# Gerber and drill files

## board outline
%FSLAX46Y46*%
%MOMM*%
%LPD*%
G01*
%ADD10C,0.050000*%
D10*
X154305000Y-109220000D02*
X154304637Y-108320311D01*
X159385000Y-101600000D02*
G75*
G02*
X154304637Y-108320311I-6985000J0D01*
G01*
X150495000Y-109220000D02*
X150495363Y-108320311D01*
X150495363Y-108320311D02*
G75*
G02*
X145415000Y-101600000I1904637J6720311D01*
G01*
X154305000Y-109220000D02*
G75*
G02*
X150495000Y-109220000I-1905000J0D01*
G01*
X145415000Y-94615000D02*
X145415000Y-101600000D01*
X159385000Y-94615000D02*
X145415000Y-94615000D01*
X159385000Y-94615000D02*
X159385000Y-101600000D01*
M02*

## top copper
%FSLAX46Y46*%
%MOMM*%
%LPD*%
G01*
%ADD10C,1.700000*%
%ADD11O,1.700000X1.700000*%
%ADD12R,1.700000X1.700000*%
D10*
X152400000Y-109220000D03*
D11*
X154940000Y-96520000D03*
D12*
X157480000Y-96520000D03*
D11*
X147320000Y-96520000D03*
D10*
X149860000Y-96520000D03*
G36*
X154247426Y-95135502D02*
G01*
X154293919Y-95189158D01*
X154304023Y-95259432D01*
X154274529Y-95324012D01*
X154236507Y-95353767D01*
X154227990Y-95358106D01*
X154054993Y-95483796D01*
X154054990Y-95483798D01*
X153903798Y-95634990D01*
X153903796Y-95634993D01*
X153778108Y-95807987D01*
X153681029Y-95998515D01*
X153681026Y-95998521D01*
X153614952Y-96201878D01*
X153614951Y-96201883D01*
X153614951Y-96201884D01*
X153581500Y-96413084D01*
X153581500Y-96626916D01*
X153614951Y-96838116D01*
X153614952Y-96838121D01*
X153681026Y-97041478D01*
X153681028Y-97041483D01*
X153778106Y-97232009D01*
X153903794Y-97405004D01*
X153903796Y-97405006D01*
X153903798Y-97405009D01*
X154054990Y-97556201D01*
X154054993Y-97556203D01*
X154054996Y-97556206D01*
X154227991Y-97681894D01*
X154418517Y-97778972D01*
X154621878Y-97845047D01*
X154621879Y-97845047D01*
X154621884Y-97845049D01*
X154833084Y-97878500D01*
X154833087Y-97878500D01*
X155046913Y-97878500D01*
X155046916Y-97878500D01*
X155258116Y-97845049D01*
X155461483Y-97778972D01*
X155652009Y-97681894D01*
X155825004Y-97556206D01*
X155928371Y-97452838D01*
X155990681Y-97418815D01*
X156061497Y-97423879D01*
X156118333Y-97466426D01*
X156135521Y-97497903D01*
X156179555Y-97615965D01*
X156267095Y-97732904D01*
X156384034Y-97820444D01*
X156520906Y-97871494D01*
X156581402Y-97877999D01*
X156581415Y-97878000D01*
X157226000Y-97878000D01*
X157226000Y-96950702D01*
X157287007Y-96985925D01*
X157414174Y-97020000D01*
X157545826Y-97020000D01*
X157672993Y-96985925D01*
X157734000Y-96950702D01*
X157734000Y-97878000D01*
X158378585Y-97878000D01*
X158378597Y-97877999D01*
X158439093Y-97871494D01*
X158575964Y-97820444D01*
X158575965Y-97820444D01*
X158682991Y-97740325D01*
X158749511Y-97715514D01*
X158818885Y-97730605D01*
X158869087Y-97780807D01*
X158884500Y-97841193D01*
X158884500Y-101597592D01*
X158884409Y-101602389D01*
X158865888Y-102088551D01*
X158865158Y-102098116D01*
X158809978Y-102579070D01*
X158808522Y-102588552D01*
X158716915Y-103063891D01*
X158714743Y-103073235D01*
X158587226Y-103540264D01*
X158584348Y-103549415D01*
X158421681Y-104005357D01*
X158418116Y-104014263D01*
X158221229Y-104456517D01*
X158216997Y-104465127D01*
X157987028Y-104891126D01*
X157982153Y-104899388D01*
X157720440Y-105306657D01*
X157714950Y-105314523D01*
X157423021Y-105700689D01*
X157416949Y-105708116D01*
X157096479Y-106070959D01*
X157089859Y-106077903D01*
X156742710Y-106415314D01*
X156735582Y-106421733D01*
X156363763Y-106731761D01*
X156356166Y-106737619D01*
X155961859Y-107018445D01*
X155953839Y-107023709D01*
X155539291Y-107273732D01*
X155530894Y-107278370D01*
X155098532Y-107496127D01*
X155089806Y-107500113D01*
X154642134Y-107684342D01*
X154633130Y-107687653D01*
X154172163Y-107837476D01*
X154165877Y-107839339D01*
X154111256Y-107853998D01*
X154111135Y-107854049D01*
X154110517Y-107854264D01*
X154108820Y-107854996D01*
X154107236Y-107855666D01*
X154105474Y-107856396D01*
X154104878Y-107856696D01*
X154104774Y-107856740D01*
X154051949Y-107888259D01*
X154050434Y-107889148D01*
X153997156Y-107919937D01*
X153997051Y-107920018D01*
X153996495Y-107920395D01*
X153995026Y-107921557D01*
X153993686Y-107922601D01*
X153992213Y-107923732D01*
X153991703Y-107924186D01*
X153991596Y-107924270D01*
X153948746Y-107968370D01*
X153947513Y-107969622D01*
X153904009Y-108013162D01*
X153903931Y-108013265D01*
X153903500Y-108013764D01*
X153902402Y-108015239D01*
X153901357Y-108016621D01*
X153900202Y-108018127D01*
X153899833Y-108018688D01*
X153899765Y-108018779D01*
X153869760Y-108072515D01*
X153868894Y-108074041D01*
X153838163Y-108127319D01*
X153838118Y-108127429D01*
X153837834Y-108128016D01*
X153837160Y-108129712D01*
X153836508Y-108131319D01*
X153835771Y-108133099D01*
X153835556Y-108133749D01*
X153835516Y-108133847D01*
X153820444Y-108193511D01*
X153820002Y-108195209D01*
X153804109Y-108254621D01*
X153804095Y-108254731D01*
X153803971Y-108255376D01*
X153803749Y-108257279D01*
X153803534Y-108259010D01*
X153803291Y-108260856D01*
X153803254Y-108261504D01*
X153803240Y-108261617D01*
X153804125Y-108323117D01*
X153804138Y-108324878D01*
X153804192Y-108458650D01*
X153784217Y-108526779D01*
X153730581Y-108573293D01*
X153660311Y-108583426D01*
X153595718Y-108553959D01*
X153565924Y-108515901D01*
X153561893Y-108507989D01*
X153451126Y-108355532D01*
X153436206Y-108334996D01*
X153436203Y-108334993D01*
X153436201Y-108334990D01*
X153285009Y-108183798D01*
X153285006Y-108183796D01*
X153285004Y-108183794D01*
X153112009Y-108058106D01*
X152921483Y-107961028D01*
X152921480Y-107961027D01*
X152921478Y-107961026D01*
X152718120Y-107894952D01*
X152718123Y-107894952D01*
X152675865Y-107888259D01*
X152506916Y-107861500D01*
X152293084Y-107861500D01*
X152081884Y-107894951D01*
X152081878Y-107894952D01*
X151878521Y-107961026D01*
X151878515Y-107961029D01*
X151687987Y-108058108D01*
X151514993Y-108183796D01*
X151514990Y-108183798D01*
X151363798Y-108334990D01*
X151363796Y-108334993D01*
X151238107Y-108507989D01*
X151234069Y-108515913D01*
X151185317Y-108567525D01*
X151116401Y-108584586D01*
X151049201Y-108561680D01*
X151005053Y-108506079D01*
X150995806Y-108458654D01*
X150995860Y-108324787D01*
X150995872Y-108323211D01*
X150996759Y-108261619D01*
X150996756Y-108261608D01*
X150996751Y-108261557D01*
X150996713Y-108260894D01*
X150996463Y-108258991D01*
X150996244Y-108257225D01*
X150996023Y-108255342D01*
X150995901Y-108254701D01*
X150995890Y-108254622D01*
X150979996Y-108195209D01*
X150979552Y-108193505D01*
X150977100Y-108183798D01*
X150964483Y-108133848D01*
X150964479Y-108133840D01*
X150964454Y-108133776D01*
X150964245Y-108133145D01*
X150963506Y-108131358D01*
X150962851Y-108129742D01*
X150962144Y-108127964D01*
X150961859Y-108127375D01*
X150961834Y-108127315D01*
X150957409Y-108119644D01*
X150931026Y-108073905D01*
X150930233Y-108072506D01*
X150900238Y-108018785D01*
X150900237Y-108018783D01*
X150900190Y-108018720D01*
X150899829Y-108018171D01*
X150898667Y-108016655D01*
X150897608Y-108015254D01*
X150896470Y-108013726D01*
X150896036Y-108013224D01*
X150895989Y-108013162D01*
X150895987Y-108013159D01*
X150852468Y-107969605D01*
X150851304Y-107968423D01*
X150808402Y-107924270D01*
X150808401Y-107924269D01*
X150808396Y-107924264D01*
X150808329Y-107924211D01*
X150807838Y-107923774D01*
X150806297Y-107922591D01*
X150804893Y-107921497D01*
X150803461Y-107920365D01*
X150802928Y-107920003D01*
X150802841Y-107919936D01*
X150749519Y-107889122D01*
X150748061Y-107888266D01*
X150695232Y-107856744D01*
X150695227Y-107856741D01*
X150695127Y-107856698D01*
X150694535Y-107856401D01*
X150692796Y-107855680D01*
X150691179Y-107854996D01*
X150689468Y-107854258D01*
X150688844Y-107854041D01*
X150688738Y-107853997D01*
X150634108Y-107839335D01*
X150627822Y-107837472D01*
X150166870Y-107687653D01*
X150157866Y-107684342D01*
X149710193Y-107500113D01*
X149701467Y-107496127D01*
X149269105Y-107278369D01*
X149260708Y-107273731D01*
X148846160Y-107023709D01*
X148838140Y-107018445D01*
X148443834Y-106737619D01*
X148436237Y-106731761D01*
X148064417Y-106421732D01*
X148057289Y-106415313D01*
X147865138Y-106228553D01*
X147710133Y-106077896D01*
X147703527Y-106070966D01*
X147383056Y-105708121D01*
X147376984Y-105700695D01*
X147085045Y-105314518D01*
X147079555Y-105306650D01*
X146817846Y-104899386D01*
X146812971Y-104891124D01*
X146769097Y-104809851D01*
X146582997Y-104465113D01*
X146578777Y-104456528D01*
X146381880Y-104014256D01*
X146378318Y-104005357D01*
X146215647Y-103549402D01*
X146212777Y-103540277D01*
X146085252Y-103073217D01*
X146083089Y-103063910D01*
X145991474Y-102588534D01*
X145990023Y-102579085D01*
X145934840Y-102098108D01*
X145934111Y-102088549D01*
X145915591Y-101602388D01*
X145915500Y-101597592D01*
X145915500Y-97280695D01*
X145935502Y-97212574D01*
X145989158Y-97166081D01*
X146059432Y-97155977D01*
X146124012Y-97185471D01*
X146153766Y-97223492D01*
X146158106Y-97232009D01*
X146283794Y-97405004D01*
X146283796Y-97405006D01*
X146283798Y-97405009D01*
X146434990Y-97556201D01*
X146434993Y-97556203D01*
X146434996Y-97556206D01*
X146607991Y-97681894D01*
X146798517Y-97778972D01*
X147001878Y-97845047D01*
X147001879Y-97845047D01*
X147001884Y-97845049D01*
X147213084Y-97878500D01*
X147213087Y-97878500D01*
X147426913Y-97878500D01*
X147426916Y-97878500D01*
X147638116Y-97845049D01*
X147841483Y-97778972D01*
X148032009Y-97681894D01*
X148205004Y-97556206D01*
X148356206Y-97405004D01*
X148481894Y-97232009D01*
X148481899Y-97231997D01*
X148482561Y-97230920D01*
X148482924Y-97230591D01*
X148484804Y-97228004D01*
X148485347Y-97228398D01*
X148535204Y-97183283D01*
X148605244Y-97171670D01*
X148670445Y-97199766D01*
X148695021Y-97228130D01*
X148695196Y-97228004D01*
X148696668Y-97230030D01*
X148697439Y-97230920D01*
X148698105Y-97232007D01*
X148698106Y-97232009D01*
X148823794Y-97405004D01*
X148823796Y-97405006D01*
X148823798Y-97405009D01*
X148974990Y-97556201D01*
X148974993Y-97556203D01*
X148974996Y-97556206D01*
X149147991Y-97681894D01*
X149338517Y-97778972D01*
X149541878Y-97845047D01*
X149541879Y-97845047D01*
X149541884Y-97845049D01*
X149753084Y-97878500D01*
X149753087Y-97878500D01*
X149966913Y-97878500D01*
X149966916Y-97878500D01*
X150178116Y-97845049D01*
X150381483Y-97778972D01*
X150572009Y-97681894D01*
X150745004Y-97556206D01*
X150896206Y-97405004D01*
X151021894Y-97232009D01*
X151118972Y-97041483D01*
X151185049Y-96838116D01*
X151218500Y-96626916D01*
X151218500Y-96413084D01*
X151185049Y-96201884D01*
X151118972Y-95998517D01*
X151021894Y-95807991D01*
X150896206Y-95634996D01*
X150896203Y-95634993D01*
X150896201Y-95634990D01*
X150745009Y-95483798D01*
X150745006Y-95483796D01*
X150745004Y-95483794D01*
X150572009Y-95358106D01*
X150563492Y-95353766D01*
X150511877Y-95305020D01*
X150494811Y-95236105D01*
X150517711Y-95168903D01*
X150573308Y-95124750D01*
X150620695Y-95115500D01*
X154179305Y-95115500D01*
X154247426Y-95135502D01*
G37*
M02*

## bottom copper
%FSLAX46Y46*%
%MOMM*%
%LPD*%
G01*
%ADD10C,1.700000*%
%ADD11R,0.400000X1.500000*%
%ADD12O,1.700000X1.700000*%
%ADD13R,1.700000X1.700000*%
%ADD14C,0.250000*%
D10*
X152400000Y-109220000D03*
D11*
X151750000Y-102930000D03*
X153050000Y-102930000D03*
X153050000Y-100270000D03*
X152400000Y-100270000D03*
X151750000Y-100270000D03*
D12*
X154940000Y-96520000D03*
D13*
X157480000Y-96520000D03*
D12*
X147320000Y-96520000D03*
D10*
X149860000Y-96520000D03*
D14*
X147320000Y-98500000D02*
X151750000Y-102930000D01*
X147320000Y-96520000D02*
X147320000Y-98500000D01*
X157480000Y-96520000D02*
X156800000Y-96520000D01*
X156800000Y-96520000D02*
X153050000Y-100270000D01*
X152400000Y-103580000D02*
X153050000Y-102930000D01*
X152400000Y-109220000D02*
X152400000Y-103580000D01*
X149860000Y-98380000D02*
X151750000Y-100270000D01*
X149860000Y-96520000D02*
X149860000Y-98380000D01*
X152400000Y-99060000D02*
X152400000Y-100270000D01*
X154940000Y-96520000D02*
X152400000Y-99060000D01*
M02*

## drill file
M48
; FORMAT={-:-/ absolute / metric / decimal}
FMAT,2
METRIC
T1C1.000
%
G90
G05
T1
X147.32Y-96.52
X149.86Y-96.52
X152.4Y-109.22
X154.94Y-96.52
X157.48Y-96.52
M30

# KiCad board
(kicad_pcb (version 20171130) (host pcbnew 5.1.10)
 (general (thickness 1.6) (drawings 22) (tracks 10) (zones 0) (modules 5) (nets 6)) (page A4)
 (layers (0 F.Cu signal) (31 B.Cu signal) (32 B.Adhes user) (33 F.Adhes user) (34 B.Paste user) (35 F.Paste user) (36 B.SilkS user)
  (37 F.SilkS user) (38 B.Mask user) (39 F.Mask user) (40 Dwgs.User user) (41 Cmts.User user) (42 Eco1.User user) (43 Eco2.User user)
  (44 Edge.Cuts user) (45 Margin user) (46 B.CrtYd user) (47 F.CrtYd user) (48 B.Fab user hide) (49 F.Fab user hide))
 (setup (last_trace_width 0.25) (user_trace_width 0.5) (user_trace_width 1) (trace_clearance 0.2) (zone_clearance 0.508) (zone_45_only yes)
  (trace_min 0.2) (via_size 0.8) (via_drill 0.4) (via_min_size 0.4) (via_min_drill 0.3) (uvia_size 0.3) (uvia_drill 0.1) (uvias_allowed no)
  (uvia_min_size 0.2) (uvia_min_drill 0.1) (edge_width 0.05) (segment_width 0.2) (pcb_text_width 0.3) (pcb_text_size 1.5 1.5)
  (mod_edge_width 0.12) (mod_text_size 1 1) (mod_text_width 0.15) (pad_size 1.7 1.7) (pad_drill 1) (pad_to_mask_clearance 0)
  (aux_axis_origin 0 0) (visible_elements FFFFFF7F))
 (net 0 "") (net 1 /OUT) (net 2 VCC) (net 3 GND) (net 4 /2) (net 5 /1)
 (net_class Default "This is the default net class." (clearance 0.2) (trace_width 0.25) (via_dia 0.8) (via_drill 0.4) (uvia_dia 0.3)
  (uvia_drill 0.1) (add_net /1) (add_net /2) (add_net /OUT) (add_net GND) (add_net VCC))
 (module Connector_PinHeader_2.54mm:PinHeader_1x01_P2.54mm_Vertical (layer B.Cu) (at 152.4 109.22 270)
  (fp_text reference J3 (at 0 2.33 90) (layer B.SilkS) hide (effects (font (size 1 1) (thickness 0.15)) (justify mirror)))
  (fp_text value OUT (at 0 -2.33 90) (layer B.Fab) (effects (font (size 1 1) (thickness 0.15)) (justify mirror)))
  (pad 1 thru_hole circle (at 0 0 270) (size 1.7 1.7) (drill 1) (layers *.Cu *.Mask) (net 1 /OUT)))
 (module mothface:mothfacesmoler (layer B.Cu) (at 155.575 102.87 255)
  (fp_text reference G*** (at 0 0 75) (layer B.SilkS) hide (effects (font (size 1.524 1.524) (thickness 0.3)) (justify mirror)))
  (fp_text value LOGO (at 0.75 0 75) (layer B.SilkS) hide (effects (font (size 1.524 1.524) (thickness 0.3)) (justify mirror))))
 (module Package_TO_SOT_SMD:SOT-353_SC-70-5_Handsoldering (layer B.Cu) (at 152.4 101.6 270)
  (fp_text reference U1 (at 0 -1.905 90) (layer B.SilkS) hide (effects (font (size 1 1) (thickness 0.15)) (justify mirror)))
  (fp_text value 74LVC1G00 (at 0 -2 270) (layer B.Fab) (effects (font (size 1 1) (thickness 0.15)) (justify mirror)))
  (pad 5 smd rect (at 1.33 0.65 270) (size 1.5 0.4) (layers B.Cu B.Paste B.Mask) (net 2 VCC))
  (pad 4 smd rect (at 1.33 -0.65 270) (size 1.5 0.4) (layers B.Cu B.Paste B.Mask) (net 1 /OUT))
  (pad 3 smd rect (at -1.33 -0.65 270) (size 1.5 0.4) (layers B.Cu B.Paste B.Mask) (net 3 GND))
  (pad 2 smd rect (at -1.33 0 270) (size 1.5 0.4) (layers B.Cu B.Paste B.Mask) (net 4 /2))
  (pad 1 smd rect (at -1.33 0.65 270) (size 1.5 0.4) (layers B.Cu B.Paste B.Mask) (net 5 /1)))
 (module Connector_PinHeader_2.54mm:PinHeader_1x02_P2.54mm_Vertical (layer B.Cu) (at 157.48 96.52 90)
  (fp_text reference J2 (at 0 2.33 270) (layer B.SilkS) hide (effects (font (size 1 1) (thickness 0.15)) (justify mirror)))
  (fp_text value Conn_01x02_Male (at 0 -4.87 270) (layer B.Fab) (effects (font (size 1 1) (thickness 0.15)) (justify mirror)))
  (pad 2 thru_hole oval (at 0 -2.54 90) (size 1.7 1.7) (drill 1) (layers *.Cu *.Mask) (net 4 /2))
  (pad 1 thru_hole rect (at 0 0 90) (size 1.7 1.7) (drill 1) (layers *.Cu *.Mask) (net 3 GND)))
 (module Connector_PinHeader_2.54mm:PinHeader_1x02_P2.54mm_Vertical (layer B.Cu) (at 149.86 96.52 90)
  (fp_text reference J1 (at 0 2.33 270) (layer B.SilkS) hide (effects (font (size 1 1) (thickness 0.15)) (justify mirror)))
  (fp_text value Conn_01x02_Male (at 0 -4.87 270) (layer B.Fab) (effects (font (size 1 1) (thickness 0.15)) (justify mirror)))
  (pad 2 thru_hole oval (at 0 -2.54 90) (size 1.7 1.7) (drill 1) (layers *.Cu *.Mask) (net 2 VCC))
  (pad 1 thru_hole circle (at 0 0 90) (size 1.7 1.7) (drill 1) (layers *.Cu *.Mask) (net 5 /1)))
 (gr_line (start 154.305 109.22) (end 154.304637 108.320311) (layer Edge.Cuts) (width 0.05))
 (gr_arc (start 152.4 101.6) (end 159.385 101.6) (angle 74.17647245) (layer Edge.Cuts) (width 0.05))
 (gr_line (start 150.495 109.22) (end 150.495363 108.320311) (layer Edge.Cuts) (width 0.05))
 (gr_arc (start 152.4 101.6) (end 145.415 101.6) (angle -74.17647245) (layer Edge.Cuts) (width 0.05))
 (gr_arc (start 152.4 109.22) (end 150.495 109.22) (angle -180) (layer Edge.Cuts) (width 0.05))
 (gr_line (start 145.415 94.615) (end 145.415 101.6) (layer Edge.Cuts) (width 0.05))
 (gr_line (start 159.385 94.615) (end 145.415 94.615) (layer Edge.Cuts) (width 0.05))
 (gr_line (start 159.385 94.615) (end 159.385 101.6) (layer Edge.Cuts) (width 0.05))
 (segment (start 147.32 98.5) (end 151.75 102.93) (width 0.25) (layer B.Cu) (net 2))
 (segment (start 147.32 96.52) (end 147.32 98.5) (width 0.25) (layer B.Cu) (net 2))
 (segment (start 157.48 96.52) (end 156.8 96.52) (width 0.25) (layer B.Cu) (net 3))
 (segment (start 156.8 96.52) (end 153.05 100.27) (width 0.25) (layer B.Cu) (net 3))
 (segment (start 152.4 103.58) (end 153.05 102.93) (width 0.25) (layer B.Cu) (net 1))
 (segment (start 152.4 109.22) (end 152.4 103.58) (width 0.25) (layer B.Cu) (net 1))
 (segment (start 149.86 98.38) (end 151.75 100.27) (width 0.25) (layer B.Cu) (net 5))
 (segment (start 149.86 96.52) (end 149.86 98.38) (width 0.25) (layer B.Cu) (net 5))
 (segment (start 152.4 99.06) (end 152.4 100.27) (width 0.25) (layer B.Cu) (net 4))
 (segment (start 154.94 96.52) (end 152.4 99.06) (width 0.25) (layer B.Cu) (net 4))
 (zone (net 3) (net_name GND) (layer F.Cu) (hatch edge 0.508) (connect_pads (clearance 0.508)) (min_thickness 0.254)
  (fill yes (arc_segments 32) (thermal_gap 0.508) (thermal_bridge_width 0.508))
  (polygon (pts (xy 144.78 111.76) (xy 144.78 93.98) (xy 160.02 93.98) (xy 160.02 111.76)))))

